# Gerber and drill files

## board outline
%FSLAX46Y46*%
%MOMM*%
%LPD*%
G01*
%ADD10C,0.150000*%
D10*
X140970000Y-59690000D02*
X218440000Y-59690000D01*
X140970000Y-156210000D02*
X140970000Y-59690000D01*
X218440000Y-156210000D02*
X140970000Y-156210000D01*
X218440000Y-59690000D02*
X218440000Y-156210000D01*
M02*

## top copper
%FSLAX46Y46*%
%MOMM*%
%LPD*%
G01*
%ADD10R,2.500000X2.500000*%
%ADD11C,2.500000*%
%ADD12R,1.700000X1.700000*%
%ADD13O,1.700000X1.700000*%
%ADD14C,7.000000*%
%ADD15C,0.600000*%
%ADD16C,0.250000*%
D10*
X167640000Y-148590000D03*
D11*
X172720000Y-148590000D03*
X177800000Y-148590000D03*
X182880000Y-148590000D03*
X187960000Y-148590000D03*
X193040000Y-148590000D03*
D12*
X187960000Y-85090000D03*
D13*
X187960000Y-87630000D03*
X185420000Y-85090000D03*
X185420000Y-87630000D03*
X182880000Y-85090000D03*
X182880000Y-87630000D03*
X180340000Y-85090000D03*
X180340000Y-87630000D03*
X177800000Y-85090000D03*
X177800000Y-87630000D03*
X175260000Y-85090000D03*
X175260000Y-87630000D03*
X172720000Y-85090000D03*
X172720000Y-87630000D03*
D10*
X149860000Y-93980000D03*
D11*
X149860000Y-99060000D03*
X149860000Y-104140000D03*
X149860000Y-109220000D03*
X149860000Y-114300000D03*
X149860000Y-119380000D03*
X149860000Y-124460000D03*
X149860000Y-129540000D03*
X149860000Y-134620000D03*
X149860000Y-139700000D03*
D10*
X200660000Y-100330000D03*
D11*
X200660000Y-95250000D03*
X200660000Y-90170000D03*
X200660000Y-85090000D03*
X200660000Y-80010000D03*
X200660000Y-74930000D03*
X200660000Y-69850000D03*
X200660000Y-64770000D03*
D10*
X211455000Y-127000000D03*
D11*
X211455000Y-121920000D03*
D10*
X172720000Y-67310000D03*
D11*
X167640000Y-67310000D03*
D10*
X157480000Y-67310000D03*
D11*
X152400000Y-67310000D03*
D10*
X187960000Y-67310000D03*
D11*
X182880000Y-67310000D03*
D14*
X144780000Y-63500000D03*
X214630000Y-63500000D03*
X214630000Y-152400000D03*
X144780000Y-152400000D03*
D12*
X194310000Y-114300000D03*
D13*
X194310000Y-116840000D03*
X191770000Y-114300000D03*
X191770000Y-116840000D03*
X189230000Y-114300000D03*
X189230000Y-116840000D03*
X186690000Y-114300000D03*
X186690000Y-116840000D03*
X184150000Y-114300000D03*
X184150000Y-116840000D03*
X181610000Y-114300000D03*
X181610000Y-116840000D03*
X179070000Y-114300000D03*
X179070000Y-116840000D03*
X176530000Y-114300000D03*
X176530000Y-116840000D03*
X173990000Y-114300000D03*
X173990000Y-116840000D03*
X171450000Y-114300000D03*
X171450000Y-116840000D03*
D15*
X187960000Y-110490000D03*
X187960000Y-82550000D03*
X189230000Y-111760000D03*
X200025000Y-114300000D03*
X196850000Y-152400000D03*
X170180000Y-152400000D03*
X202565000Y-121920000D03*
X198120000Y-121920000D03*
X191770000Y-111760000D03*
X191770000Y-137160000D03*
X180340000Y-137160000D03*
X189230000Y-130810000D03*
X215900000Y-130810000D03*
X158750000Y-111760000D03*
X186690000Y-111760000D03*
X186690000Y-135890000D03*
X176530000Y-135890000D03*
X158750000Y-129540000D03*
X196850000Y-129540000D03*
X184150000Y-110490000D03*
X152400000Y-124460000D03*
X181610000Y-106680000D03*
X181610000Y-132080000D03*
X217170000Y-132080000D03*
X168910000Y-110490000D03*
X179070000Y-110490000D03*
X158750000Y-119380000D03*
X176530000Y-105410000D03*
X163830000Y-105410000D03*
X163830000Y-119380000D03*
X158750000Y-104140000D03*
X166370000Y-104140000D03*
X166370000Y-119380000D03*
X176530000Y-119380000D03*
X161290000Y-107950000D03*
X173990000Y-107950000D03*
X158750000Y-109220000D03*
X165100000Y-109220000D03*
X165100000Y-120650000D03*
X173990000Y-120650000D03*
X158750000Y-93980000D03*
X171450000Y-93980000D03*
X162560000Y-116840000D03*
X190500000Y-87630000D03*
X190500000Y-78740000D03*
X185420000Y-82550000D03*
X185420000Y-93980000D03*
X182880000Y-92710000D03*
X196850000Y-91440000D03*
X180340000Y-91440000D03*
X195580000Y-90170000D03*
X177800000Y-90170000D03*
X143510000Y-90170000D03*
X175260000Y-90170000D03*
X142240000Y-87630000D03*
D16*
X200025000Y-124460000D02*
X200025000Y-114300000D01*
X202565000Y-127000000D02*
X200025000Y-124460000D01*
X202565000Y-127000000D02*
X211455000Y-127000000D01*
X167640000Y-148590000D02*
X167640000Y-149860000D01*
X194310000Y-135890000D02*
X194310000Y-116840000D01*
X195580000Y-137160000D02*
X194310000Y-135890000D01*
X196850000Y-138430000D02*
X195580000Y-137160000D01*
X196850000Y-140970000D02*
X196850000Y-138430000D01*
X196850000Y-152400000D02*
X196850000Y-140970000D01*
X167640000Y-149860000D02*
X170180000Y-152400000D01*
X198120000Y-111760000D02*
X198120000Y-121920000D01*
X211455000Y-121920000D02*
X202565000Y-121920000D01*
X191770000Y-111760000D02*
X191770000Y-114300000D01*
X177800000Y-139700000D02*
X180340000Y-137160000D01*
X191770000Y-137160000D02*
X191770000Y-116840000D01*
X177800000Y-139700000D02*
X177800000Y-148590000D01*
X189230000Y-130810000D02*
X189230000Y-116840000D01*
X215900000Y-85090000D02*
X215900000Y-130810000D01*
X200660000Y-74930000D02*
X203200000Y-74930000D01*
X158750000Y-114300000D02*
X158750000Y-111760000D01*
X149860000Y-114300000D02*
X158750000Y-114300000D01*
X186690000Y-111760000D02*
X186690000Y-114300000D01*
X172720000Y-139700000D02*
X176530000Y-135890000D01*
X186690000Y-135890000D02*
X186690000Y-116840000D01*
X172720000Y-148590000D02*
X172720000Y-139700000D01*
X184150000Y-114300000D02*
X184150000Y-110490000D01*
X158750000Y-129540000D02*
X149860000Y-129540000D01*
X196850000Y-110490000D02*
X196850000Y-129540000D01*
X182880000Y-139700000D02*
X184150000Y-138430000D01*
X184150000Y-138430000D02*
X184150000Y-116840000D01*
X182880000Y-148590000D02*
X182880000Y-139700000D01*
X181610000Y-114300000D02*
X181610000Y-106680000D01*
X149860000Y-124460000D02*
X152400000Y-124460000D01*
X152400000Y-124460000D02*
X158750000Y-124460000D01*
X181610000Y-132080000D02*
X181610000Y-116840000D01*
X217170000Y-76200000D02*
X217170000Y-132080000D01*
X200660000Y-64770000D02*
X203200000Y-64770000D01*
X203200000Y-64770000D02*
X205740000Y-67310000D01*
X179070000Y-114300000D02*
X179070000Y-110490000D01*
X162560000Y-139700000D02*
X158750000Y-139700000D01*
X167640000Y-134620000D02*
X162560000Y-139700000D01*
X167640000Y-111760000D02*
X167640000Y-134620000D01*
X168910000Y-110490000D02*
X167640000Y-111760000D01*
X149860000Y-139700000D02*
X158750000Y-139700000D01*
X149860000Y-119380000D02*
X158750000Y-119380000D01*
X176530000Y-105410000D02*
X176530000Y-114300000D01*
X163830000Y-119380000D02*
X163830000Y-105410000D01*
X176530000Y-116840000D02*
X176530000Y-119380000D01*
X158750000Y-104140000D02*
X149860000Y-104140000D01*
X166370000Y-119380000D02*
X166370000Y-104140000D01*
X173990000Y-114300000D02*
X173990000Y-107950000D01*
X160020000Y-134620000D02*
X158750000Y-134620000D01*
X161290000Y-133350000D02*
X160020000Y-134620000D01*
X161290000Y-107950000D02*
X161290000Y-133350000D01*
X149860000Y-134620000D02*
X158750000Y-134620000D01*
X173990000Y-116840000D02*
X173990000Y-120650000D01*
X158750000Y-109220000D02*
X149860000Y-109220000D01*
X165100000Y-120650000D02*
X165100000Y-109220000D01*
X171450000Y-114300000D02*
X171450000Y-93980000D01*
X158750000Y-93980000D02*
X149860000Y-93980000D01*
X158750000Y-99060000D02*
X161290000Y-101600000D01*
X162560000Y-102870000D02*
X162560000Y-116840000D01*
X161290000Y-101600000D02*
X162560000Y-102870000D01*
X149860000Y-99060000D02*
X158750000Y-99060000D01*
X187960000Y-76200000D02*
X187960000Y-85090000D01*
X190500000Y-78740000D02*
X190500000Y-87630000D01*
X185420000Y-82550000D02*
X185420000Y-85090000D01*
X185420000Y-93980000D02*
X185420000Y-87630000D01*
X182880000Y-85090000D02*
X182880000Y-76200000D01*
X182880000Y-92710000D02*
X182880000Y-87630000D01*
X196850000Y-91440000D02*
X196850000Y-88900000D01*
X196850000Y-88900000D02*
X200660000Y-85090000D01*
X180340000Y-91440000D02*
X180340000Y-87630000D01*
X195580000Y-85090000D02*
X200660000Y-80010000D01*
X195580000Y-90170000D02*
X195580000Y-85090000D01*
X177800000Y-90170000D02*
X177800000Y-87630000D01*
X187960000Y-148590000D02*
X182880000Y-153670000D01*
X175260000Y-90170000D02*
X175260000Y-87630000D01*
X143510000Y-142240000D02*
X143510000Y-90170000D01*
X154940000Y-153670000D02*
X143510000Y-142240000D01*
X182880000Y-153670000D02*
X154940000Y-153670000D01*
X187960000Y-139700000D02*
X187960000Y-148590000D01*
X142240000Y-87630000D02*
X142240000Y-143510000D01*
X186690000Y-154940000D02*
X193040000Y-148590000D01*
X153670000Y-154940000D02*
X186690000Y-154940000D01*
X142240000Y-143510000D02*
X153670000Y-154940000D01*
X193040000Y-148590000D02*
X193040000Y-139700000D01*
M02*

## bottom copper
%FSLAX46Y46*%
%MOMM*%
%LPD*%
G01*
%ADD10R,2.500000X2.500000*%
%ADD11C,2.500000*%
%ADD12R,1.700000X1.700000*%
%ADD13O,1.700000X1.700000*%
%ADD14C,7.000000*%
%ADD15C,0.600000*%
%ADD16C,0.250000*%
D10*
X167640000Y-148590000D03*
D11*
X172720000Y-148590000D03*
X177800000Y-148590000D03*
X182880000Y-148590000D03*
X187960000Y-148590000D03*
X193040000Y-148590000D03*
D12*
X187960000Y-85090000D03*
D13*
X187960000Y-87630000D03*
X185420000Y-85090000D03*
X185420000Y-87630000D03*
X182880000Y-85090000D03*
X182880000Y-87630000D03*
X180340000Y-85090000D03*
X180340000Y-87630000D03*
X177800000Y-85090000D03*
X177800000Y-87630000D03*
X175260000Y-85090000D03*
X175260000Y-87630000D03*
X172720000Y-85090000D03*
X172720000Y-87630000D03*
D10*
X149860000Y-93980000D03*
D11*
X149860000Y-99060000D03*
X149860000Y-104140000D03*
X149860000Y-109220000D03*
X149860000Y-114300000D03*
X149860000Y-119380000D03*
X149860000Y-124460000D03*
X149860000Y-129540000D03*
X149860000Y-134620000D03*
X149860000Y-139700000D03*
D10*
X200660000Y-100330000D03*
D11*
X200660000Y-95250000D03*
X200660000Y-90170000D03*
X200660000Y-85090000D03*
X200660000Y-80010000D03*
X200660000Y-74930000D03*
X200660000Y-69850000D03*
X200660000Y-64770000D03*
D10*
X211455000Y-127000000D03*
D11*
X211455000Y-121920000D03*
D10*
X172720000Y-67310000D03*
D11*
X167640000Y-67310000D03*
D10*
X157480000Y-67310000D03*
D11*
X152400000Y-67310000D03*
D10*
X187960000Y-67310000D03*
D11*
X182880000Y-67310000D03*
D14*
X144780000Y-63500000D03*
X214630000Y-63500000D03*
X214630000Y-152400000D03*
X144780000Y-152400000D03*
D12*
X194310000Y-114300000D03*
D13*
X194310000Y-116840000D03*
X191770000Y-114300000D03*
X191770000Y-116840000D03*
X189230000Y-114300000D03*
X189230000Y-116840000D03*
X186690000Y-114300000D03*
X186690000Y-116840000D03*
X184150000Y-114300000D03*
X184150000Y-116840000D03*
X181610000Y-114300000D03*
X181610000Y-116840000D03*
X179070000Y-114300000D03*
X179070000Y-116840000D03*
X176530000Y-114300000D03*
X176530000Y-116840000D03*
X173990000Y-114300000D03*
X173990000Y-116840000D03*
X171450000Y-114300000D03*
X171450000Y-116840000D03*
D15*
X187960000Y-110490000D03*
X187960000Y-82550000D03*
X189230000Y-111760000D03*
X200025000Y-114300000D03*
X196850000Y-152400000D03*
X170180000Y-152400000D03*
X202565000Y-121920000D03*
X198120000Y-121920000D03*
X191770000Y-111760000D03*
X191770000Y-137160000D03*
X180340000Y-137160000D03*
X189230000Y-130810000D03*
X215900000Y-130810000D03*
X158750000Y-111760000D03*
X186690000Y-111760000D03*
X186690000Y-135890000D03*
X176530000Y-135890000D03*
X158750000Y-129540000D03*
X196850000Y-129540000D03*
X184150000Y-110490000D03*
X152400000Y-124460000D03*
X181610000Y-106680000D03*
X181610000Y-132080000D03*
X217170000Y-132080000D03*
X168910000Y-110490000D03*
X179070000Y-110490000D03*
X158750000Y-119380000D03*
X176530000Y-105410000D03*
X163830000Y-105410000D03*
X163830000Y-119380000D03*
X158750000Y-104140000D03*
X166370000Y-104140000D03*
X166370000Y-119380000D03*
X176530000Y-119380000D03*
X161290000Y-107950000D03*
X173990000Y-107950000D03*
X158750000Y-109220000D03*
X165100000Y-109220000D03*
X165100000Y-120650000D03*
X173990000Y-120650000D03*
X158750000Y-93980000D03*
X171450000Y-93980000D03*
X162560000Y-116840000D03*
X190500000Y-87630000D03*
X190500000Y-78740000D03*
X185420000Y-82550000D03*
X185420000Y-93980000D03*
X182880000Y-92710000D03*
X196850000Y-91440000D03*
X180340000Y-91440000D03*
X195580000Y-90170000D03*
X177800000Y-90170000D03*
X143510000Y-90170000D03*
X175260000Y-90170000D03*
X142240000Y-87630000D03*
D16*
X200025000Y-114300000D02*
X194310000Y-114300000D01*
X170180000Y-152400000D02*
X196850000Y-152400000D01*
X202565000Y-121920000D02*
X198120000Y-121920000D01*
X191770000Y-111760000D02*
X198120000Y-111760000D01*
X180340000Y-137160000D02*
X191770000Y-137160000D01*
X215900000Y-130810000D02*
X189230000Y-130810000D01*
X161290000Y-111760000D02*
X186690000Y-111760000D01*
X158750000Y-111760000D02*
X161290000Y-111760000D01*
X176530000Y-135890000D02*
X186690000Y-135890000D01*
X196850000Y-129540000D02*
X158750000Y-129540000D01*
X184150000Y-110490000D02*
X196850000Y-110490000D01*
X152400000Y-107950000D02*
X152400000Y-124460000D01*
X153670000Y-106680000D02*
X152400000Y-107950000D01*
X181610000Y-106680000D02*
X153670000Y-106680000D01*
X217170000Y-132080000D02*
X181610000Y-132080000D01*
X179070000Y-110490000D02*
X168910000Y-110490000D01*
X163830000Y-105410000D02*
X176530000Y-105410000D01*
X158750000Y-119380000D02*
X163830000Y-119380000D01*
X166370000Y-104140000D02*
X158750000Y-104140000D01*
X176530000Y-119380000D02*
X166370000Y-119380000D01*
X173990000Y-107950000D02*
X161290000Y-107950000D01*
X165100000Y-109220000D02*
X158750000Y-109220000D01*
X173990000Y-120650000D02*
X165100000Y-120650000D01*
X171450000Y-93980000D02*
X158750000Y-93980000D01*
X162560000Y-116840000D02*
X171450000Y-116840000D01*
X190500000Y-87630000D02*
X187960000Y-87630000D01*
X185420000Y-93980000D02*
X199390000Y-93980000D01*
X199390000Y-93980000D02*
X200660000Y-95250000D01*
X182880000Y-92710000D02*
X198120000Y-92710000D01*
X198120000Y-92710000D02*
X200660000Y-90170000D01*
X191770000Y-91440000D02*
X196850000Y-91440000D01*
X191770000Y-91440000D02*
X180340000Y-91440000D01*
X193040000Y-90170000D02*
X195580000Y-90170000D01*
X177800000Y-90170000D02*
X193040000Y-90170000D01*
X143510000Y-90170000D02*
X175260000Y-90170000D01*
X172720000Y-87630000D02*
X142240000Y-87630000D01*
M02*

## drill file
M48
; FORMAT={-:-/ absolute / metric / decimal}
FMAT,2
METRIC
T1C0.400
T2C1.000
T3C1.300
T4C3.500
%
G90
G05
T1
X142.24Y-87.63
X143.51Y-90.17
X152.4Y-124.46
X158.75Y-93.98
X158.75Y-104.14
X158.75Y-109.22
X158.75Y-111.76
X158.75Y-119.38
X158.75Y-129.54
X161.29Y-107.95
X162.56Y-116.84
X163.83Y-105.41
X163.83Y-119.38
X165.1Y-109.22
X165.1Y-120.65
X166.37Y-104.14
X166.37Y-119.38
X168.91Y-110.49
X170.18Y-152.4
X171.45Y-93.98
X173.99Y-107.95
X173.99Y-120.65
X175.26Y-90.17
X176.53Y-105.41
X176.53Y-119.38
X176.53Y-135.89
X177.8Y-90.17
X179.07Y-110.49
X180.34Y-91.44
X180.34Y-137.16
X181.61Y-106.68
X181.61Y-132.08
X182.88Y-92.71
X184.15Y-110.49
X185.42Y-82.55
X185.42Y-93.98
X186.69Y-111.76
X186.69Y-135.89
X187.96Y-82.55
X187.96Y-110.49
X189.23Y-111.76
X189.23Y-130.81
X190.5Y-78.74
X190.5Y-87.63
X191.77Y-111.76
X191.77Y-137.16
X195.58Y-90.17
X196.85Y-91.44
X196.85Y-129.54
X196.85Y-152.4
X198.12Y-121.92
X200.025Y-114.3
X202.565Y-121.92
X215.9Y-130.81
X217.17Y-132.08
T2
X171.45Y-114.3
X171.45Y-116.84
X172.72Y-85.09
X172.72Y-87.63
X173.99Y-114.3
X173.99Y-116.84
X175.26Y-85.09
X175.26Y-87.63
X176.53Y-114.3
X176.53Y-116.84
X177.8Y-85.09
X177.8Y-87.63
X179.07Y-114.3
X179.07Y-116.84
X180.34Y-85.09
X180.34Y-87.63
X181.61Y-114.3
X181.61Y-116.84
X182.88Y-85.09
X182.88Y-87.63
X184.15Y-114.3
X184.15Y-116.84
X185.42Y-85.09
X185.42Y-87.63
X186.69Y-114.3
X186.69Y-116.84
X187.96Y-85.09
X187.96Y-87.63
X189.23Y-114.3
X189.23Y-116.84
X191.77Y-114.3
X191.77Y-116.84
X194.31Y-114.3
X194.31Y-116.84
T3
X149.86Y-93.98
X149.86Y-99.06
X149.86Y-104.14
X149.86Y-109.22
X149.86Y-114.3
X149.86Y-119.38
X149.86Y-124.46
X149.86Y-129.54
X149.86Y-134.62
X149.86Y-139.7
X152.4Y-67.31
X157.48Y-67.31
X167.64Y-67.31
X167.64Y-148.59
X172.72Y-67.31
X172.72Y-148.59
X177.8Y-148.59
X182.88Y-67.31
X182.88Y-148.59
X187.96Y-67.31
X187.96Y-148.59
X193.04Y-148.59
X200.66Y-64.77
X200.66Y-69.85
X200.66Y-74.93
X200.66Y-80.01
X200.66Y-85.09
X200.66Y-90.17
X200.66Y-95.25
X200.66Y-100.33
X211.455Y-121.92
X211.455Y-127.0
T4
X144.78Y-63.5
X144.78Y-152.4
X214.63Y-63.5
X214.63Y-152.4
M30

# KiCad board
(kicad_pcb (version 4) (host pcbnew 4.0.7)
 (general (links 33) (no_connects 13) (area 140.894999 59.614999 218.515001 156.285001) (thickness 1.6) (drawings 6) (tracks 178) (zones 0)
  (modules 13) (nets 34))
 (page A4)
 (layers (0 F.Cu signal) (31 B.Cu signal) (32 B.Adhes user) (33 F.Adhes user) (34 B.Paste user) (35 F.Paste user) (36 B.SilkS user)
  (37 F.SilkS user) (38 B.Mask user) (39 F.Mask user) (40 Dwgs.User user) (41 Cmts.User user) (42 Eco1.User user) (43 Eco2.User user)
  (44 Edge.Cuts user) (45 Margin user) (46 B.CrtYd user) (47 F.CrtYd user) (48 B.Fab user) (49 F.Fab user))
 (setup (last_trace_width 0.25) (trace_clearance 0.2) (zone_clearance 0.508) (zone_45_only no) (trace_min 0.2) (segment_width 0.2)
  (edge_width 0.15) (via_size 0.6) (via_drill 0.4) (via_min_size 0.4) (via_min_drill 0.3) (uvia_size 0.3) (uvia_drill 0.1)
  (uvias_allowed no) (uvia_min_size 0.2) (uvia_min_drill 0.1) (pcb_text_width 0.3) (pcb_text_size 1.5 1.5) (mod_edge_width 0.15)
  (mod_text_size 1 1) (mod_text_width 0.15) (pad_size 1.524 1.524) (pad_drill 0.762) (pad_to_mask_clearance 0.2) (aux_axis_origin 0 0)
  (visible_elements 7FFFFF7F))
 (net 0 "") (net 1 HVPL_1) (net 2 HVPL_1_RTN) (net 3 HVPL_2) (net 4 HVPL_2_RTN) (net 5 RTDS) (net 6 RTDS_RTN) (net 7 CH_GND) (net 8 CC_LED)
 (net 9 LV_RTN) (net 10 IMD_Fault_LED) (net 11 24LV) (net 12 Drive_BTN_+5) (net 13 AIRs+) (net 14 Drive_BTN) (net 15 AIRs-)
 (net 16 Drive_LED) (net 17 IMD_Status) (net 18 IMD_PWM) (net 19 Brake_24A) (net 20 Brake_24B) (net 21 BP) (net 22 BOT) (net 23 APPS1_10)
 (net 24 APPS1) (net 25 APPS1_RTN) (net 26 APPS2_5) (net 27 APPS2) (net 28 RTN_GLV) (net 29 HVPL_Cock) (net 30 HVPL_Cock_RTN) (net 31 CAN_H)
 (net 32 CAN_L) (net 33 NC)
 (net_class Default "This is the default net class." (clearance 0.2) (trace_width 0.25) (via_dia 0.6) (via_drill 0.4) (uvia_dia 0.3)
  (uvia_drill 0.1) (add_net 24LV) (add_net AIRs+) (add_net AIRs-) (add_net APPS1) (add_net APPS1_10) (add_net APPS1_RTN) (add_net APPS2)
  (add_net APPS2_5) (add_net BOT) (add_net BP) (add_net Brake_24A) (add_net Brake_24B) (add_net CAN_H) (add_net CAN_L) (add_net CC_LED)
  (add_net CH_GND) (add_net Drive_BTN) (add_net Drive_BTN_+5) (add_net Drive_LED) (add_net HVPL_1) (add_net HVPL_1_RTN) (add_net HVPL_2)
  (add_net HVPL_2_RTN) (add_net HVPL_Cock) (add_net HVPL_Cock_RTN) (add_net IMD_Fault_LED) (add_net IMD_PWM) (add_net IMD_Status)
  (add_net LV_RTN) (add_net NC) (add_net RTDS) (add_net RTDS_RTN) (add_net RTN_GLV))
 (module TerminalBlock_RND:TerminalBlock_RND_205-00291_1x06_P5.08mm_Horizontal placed (layer F.Cu) (at 167.64 148.59)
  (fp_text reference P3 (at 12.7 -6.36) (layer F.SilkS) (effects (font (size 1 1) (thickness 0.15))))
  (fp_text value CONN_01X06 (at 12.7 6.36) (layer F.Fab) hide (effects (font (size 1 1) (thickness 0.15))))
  (pad 1 thru_hole rect (at 0 0) (size 2.5 2.5) (drill 1.3) (layers *.Cu *.Mask) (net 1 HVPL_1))
  (pad 2 thru_hole circle (at 5.08 0) (size 2.5 2.5) (drill 1.3) (layers *.Cu *.Mask) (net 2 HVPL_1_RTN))
  (pad 3 thru_hole circle (at 10.16 0) (size 2.5 2.5) (drill 1.3) (layers *.Cu *.Mask) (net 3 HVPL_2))
  (pad 4 thru_hole circle (at 15.24 0) (size 2.5 2.5) (drill 1.3) (layers *.Cu *.Mask) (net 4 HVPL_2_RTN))
  (pad 5 thru_hole circle (at 20.32 0) (size 2.5 2.5) (drill 1.3) (layers *.Cu *.Mask) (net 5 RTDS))
  (pad 6 thru_hole circle (at 25.4 0) (size 2.5 2.5) (drill 1.3) (layers *.Cu *.Mask) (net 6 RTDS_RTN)))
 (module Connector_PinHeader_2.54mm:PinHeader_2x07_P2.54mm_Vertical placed (layer F.Cu) (at 187.96 85.09 270)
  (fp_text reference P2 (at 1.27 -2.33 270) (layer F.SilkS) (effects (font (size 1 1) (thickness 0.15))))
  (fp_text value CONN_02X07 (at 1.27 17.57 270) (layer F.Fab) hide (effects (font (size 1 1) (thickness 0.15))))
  (pad 1 thru_hole rect (at 0 0 270) (size 1.7 1.7) (drill 1) (layers *.Cu *.Mask) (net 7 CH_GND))
  (pad 2 thru_hole oval (at 2.54 0 270) (size 1.7 1.7) (drill 1) (layers *.Cu *.Mask) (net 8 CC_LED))
  (pad 3 thru_hole oval (at 0 2.54 270) (size 1.7 1.7) (drill 1) (layers *.Cu *.Mask) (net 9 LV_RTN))
  (pad 4 thru_hole oval (at 2.54 2.54 270) (size 1.7 1.7) (drill 1) (layers *.Cu *.Mask) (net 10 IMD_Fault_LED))
  (pad 5 thru_hole oval (at 0 5.08 270) (size 1.7 1.7) (drill 1) (layers *.Cu *.Mask) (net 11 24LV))
  (pad 6 thru_hole oval (at 2.54 5.08 270) (size 1.7 1.7) (drill 1) (layers *.Cu *.Mask) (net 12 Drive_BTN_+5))
  (pad 7 thru_hole oval (at 0 7.62 270) (size 1.7 1.7) (drill 1) (layers *.Cu *.Mask) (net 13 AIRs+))
  (pad 8 thru_hole oval (at 2.54 7.62 270) (size 1.7 1.7) (drill 1) (layers *.Cu *.Mask) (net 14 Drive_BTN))
  (pad 9 thru_hole oval (at 0 10.16 270) (size 1.7 1.7) (drill 1) (layers *.Cu *.Mask) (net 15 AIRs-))
  (pad 10 thru_hole oval (at 2.54 10.16 270) (size 1.7 1.7) (drill 1) (layers *.Cu *.Mask) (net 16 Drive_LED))
  (pad 11 thru_hole oval (at 0 12.7 270) (size 1.7 1.7) (drill 1) (layers *.Cu *.Mask) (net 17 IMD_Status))
  (pad 12 thru_hole oval (at 2.54 12.7 270) (size 1.7 1.7) (drill 1) (layers *.Cu *.Mask) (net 5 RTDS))
  (pad 13 thru_hole oval (at 0 15.24 270) (size 1.7 1.7) (drill 1) (layers *.Cu *.Mask) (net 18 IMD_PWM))
  (pad 14 thru_hole oval (at 2.54 15.24 270) (size 1.7 1.7) (drill 1) (layers *.Cu *.Mask) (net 6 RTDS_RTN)))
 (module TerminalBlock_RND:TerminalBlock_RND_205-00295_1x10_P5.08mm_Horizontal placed (layer F.Cu) (at 149.86 93.98 270)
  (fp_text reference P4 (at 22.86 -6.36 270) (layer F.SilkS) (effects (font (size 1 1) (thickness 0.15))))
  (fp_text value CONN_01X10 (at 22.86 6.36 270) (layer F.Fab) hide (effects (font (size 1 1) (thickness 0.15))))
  (pad 1 thru_hole rect (at 0 0 270) (size 2.5 2.5) (drill 1.3) (layers *.Cu *.Mask) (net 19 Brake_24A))
  (pad 2 thru_hole circle (at 5.08 0 270) (size 2.5 2.5) (drill 1.3) (layers *.Cu *.Mask) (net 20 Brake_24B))
  (pad 3 thru_hole circle (at 10.16 0 270) (size 2.5 2.5) (drill 1.3) (layers *.Cu *.Mask) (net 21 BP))
  (pad 4 thru_hole circle (at 15.24 0 270) (size 2.5 2.5) (drill 1.3) (layers *.Cu *.Mask) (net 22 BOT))
  (pad 5 thru_hole circle (at 20.32 0 270) (size 2.5 2.5) (drill 1.3) (layers *.Cu *.Mask) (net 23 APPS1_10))
  (pad 6 thru_hole circle (at 25.4 0 270) (size 2.5 2.5) (drill 1.3) (layers *.Cu *.Mask) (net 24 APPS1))
  (pad 7 thru_hole circle (at 30.48 0 270) (size 2.5 2.5) (drill 1.3) (layers *.Cu *.Mask) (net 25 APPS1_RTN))
  (pad 8 thru_hole circle (at 35.56 0 270) (size 2.5 2.5) (drill 1.3) (layers *.Cu *.Mask) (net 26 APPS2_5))
  (pad 9 thru_hole circle (at 40.64 0 270) (size 2.5 2.5) (drill 1.3) (layers *.Cu *.Mask) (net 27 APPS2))
  (pad 10 thru_hole circle (at 45.72 0 270) (size 2.5 2.5) (drill 1.3) (layers *.Cu *.Mask) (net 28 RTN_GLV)))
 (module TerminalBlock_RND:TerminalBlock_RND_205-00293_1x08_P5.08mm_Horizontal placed (layer F.Cu) (at 200.66 100.33 90)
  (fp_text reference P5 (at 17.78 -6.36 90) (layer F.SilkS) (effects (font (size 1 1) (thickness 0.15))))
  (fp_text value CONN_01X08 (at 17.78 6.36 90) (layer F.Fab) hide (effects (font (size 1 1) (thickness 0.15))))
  (pad 1 thru_hole rect (at 0 0 90) (size 2.5 2.5) (drill 1.3) (layers *.Cu *.Mask) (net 9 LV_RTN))
  (pad 2 thru_hole circle (at 5.08 0 90) (size 2.5 2.5) (drill 1.3) (layers *.Cu *.Mask) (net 10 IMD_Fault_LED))
  (pad 3 thru_hole circle (at 10.16 0 90) (size 2.5 2.5) (drill 1.3) (layers *.Cu *.Mask) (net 12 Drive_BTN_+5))
  (pad 4 thru_hole circle (at 15.24 0 90) (size 2.5 2.5) (drill 1.3) (layers *.Cu *.Mask) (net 14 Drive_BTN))
  (pad 5 thru_hole circle (at 20.32 0 90) (size 2.5 2.5) (drill 1.3) (layers *.Cu *.Mask) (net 16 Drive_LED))
  (pad 6 thru_hole circle (at 25.4 0 90) (size 2.5 2.5) (drill 1.3) (layers *.Cu *.Mask) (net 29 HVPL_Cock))
  (pad 7 thru_hole circle (at 30.48 0 90) (size 2.5 2.5) (drill 1.3) (layers *.Cu *.Mask) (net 8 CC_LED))
  (pad 8 thru_hole circle (at 35.56 0 90) (size 2.5 2.5) (drill 1.3) (layers *.Cu *.Mask) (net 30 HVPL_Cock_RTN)))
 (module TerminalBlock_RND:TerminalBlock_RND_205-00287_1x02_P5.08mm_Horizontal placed (layer F.Cu) (at 211.455 127 90)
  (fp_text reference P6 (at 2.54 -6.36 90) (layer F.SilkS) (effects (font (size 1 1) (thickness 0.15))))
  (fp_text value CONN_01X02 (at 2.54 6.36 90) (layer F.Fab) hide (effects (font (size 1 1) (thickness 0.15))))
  (pad 1 thru_hole rect (at 0 0 90) (size 2.5 2.5) (drill 1.3) (layers *.Cu *.Mask) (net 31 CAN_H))
  (pad 2 thru_hole circle (at 5.08 0 90) (size 2.5 2.5) (drill 1.3) (layers *.Cu *.Mask) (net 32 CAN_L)))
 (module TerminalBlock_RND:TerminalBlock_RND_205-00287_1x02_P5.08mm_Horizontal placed (layer F.Cu) (at 172.72 67.31 180)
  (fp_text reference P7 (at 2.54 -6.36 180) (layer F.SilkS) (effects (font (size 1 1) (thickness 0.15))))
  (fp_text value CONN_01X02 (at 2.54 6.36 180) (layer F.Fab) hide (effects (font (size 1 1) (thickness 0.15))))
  (pad 1 thru_hole rect (at 0 0 180) (size 2.5 2.5) (drill 1.3) (layers *.Cu *.Mask) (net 13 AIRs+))
  (pad 2 thru_hole circle (at 5.08 0 180) (size 2.5 2.5) (drill 1.3) (layers *.Cu *.Mask) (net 15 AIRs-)))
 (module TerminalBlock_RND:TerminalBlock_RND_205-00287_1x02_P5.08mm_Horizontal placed (layer F.Cu) (at 157.48 67.31 180)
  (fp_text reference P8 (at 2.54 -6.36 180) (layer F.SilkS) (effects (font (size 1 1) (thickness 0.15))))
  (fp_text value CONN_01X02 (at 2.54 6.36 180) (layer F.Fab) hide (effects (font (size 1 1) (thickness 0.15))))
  (pad 1 thru_hole rect (at 0 0 180) (size 2.5 2.5) (drill 1.3) (layers *.Cu *.Mask) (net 17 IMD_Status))
  (pad 2 thru_hole circle (at 5.08 0 180) (size 2.5 2.5) (drill 1.3) (layers *.Cu *.Mask) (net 18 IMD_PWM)))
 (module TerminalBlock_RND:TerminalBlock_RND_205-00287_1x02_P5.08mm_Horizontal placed (layer F.Cu) (at 187.96 67.31 180)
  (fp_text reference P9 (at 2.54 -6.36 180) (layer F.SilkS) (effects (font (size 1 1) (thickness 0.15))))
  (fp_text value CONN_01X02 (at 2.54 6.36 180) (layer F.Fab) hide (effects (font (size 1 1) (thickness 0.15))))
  (pad 1 thru_hole rect (at 0 0 180) (size 2.5 2.5) (drill 1.3) (layers *.Cu *.Mask) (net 7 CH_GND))
  (pad 2 thru_hole circle (at 5.08 0 180) (size 2.5 2.5) (drill 1.3) (layers *.Cu *.Mask) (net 11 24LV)))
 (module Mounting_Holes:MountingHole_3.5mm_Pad (layer F.Cu) (at 144.78 63.5)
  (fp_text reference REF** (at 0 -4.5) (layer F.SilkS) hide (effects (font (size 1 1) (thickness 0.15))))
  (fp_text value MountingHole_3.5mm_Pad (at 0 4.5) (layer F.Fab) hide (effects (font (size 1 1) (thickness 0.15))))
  (pad 1 thru_hole circle (at 0 0) (size 7 7) (drill 3.5) (layers *.Cu *.Mask)))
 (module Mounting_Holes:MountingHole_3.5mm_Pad (layer F.Cu) (at 214.63 63.5)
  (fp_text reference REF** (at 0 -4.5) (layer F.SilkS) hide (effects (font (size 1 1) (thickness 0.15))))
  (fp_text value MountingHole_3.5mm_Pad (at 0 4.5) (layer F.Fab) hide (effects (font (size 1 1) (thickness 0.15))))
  (pad 1 thru_hole circle (at 0 0) (size 7 7) (drill 3.5) (layers *.Cu *.Mask)))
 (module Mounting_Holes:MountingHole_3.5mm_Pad (layer F.Cu) (at 214.63 152.4)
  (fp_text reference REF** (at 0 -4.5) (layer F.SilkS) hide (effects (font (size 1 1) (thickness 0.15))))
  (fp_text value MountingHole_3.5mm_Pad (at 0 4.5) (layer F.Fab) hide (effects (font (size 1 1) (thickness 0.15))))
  (pad 1 thru_hole circle (at 0 0) (size 7 7) (drill 3.5) (layers *.Cu *.Mask)))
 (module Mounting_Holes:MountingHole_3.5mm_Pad (layer F.Cu) (at 144.78 152.4)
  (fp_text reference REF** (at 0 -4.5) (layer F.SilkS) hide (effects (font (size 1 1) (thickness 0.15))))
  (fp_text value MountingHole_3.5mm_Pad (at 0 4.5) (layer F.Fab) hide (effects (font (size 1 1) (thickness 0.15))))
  (pad 1 thru_hole circle (at 0 0) (size 7 7) (drill 3.5) (layers *.Cu *.Mask)))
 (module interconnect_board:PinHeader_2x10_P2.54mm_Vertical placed (layer F.Cu) (at 194.31 114.3 270)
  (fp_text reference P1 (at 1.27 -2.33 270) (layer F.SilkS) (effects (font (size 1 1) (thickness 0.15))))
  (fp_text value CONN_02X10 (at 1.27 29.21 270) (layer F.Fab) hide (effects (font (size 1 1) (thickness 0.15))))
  (pad 1 thru_hole rect (at 0 0 270) (size 1.7 1.7) (drill 1) (layers *.Cu *.Mask) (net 31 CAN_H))
  (pad 2 thru_hole oval (at 2.54 0 270) (size 1.7 1.7) (drill 1) (layers *.Cu *.Mask) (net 1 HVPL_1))
  (pad 3 thru_hole oval (at 0 2.54 270) (size 1.7 1.7) (drill 1) (layers *.Cu *.Mask) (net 32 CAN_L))
  (pad 4 thru_hole oval (at 2.54 2.54 270) (size 1.7 1.7) (drill 1) (layers *.Cu *.Mask) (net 3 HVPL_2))
  (pad 5 thru_hole oval (at 0 5.08 270) (size 1.7 1.7) (drill 1) (layers *.Cu *.Mask) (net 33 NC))
  (pad 6 thru_hole oval (at 2.54 5.08 270) (size 1.7 1.7) (drill 1) (layers *.Cu *.Mask) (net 29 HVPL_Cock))
  (pad 7 thru_hole oval (at 0 7.62 270) (size 1.7 1.7) (drill 1) (layers *.Cu *.Mask) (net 23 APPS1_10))
  (pad 8 thru_hole oval (at 2.54 7.62 270) (size 1.7 1.7) (drill 1) (layers *.Cu *.Mask) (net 2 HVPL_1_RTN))
  (pad 9 thru_hole oval (at 0 10.16 270) (size 1.7 1.7) (drill 1) (layers *.Cu *.Mask) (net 26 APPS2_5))
  (pad 10 thru_hole oval (at 2.54 10.16 270) (size 1.7 1.7) (drill 1) (layers *.Cu *.Mask) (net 4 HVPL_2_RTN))
  (pad 11 thru_hole oval (at 0 12.7 270) (size 1.7 1.7) (drill 1) (layers *.Cu *.Mask) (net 25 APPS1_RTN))
  (pad 12 thru_hole oval (at 2.54 12.7 270) (size 1.7 1.7) (drill 1) (layers *.Cu *.Mask) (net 30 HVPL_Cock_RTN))
  (pad 13 thru_hole oval (at 0 15.24 270) (size 1.7 1.7) (drill 1) (layers *.Cu *.Mask) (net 28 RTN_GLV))
  (pad 14 thru_hole oval (at 2.54 15.24 270) (size 1.7 1.7) (drill 1) (layers *.Cu *.Mask) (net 33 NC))
  (pad 15 thru_hole oval (at 0 17.78 270) (size 1.7 1.7) (drill 1) (layers *.Cu *.Mask) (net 24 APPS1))
  (pad 16 thru_hole oval (at 2.54 17.78 270) (size 1.7 1.7) (drill 1) (layers *.Cu *.Mask) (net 21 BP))
  (pad 17 thru_hole oval (at 0 20.32 270) (size 1.7 1.7) (drill 1) (layers *.Cu *.Mask) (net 27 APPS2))
  (pad 18 thru_hole oval (at 2.54 20.32 270) (size 1.7 1.7) (drill 1) (layers *.Cu *.Mask) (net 22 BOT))
  (pad 19 thru_hole oval (at 0 22.86 270) (size 1.7 1.7) (drill 1) (layers *.Cu *.Mask) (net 19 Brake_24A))
  (pad 20 thru_hole oval (at 2.54 22.86 270) (size 1.7 1.7) (drill 1) (layers *.Cu *.Mask) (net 20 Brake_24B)))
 (gr_line (start 140.97 59.69) (end 218.44 59.69) (angle 90) (layer Edge.Cuts) (width 0.15))
 (gr_line (start 140.97 156.21) (end 140.97 59.69) (angle 90) (layer Edge.Cuts) (width 0.15))
 (gr_line (start 218.44 156.21) (end 140.97 156.21) (angle 90) (layer Edge.Cuts) (width 0.15))
 (gr_line (start 218.44 59.69) (end 218.44 156.21) (angle 90) (layer Edge.Cuts) (width 0.15))
 (via (at 187.96 110.49) (size 0.6) (drill 0.4) (layers F.Cu B.Cu) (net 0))
 (via (at 187.96 82.55) (size 0.6) (drill 0.4) (layers F.Cu B.Cu) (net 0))
 (via (at 189.23 111.76) (size 0.6) (drill 0.4) (layers F.Cu B.Cu) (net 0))
 (segment (start 200.025 114.3) (end 194.31 114.3) (width 0.25) (layer B.Cu) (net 31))
 (via (at 200.025 114.3) (size 0.6) (drill 0.4) (layers F.Cu B.Cu) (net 31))
 (segment (start 200.025 124.46) (end 200.025 114.3) (width 0.25) (layer F.Cu) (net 31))
 (segment (start 202.565 127) (end 200.025 124.46) (width 0.25) (layer F.Cu) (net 31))
 (segment (start 202.565 127) (end 211.455 127) (width 0.25) (layer F.Cu) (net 31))
 (segment (start 167.64 148.59) (end 167.64 149.86) (width 0.25) (layer F.Cu) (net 1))
 (segment (start 194.31 135.89) (end 194.31 116.84) (width 0.25) (layer F.Cu) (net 1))
 (segment (start 195.58 137.16) (end 194.31 135.89) (width 0.25) (layer F.Cu) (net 1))
 (segment (start 196.85 138.43) (end 195.58 137.16) (width 0.25) (layer F.Cu) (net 1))
 (segment (start 196.85 140.97) (end 196.85 138.43) (width 0.25) (layer F.Cu) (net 1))
 (segment (start 196.85 152.4) (end 196.85 140.97) (width 0.25) (layer F.Cu) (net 1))
 (via (at 196.85 152.4) (size 0.6) (drill 0.4) (layers F.Cu B.Cu) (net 1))
 (segment (start 170.18 152.4) (end 196.85 152.4) (width 0.25) (layer B.Cu) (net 1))
 (via (at 170.18 152.4) (size 0.6) (drill 0.4) (layers F.Cu B.Cu) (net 1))
 (segment (start 167.64 149.86) (end 170.18 152.4) (width 0.25) (layer F.Cu) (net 1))
 (via (at 202.565 121.92) (size 0.6) (drill 0.4) (layers F.Cu B.Cu) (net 32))
 (segment (start 198.12 111.76) (end 198.12 121.92) (width 0.25) (layer F.Cu) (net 32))
 (via (at 198.12 121.92) (size 0.6) (drill 0.4) (layers F.Cu B.Cu) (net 32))
 (segment (start 202.565 121.92) (end 198.12 121.92) (width 0.25) (layer B.Cu) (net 32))
 (segment (start 211.455 121.92) (end 202.565 121.92) (width 0.25) (layer F.Cu) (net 32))
 (segment (start 191.77 111.76) (end 191.77 114.3) (width 0.25) (layer F.Cu) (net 32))
 (segment (start 191.77 111.76) (end 198.12 111.76) (width 0.25) (layer B.Cu) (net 32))
 (via (at 191.77 111.76) (size 0.6) (drill 0.4) (layers F.Cu B.Cu) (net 32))
 (segment (start 177.8 139.7) (end 180.34 137.16) (width 0.25) (layer F.Cu) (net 3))
 (segment (start 191.77 137.16) (end 191.77 116.84) (width 0.25) (layer F.Cu) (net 3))
 (via (at 191.77 137.16) (size 0.6) (drill 0.4) (layers F.Cu B.Cu) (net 3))
 (segment (start 180.34 137.16) (end 191.77 137.16) (width 0.25) (layer B.Cu) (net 3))
 (via (at 180.34 137.16) (size 0.6) (drill 0.4) (layers F.Cu B.Cu) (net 3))
 (segment (start 177.8 139.7) (end 177.8 148.59) (width 0.25) (layer F.Cu) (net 3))
 (segment (start 189.23 130.81) (end 189.23 116.84) (width 0.25) (layer F.Cu) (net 29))
 (via (at 189.23 130.81) (size 0.6) (drill 0.4) (layers F.Cu B.Cu) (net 29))
 (segment (start 215.9 130.81) (end 189.23 130.81) (width 0.25) (layer B.Cu) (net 29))
 (via (at 215.9 130.81) (size 0.6) (drill 0.4) (layers F.Cu B.Cu) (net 29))
 (segment (start 215.9 85.09) (end 215.9 130.81) (width 0.25) (layer F.Cu) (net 29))
 (segment (start 200.66 74.93) (end 203.2 74.93) (width 0.25) (layer F.Cu) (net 29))
 (segment (start 158.75 114.3) (end 158.75 111.76) (width 0.25) (layer F.Cu) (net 23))
 (via (at 158.75 111.76) (size 0.6) (drill 0.4) (layers F.Cu B.Cu) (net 23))
 (segment (start 149.86 114.3) (end 158.75 114.3) (width 0.25) (layer F.Cu) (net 23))
 (segment (start 161.29 111.76) (end 186.69 111.76) (width 0.25) (layer B.Cu) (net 23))
 (via (at 186.69 111.76) (size 0.6) (drill 0.4) (layers F.Cu B.Cu) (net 23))
 (segment (start 186.69 111.76) (end 186.69 114.3) (width 0.25) (layer F.Cu) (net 23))
 (segment (start 158.75 111.76) (end 161.29 111.76) (width 0.25) (layer B.Cu) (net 23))
 (segment (start 172.72 139.7) (end 176.53 135.89) (width 0.25) (layer F.Cu) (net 2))
 (segment (start 186.69 135.89) (end 186.69 116.84) (width 0.25) (layer F.Cu) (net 2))
 (via (at 186.69 135.89) (size 0.6) (drill 0.4) (layers F.Cu B.Cu) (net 2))
 (segment (start 176.53 135.89) (end 186.69 135.89) (width 0.25) (layer B.Cu) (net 2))
 (via (at 176.53 135.89) (size 0.6) (drill 0.4) (layers F.Cu B.Cu) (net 2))
 (segment (start 172.72 148.59) (end 172.72 139.7) (width 0.25) (layer F.Cu) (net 2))
 (segment (start 184.15 114.3) (end 184.15 110.49) (width 0.25) (layer F.Cu) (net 26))
 (segment (start 158.75 129.54) (end 149.86 129.54) (width 0.25) (layer F.Cu) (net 26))
 (via (at 158.75 129.54) (size 0.6) (drill 0.4) (layers F.Cu B.Cu) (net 26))
 (segment (start 196.85 129.54) (end 158.75 129.54) (width 0.25) (layer B.Cu) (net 26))
 (via (at 196.85 129.54) (size 0.6) (drill 0.4) (layers F.Cu B.Cu) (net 26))
 (segment (start 196.85 110.49) (end 196.85 129.54) (width 0.25) (layer F.Cu) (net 26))
 (segment (start 184.15 110.49) (end 196.85 110.49) (width 0.25) (layer B.Cu) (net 26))
 (via (at 184.15 110.49) (size 0.6) (drill 0.4) (layers F.Cu B.Cu) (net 26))
 (segment (start 182.88 139.7) (end 184.15 138.43) (width 0.25) (layer F.Cu) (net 4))
 (segment (start 184.15 138.43) (end 184.15 116.84) (width 0.25) (layer F.Cu) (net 4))
 (segment (start 182.88 148.59) (end 182.88 139.7) (width 0.25) (layer F.Cu) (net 4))
 (segment (start 181.61 114.3) (end 181.61 106.68) (width 0.25) (layer F.Cu) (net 25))
 (via (at 152.4 124.46) (size 0.6) (drill 0.4) (layers F.Cu B.Cu) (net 25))
 (segment (start 152.4 107.95) (end 152.4 124.46) (width 0.25) (layer B.Cu) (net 25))
 (segment (start 153.67 106.68) (end 152.4 107.95) (width 0.25) (layer B.Cu) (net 25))
 (segment (start 181.61 106.68) (end 153.67 106.68) (width 0.25) (layer B.Cu) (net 25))
 (via (at 181.61 106.68) (size 0.6) (drill 0.4) (layers F.Cu B.Cu) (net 25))
 (segment (start 149.86 124.46) (end 152.4 124.46) (width 0.25) (layer F.Cu) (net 25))
 (segment (start 152.4 124.46) (end 158.75 124.46) (width 0.25) (layer F.Cu) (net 25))
 (segment (start 181.61 132.08) (end 181.61 116.84) (width 0.25) (layer F.Cu) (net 30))
 (via (at 181.61 132.08) (size 0.6) (drill 0.4) (layers F.Cu B.Cu) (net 30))
 (segment (start 217.17 132.08) (end 181.61 132.08) (width 0.25) (layer B.Cu) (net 30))
 (via (at 217.17 132.08) (size 0.6) (drill 0.4) (layers F.Cu B.Cu) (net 30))
 (segment (start 217.17 76.2) (end 217.17 132.08) (width 0.25) (layer F.Cu) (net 30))
 (segment (start 200.66 64.77) (end 203.2 64.77) (width 0.25) (layer F.Cu) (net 30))
 (segment (start 203.2 64.77) (end 205.74 67.31) (width 0.25) (layer F.Cu) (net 30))
 (segment (start 179.07 114.3) (end 179.07 110.49) (width 0.25) (layer F.Cu) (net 28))
 (segment (start 162.56 139.7) (end 158.75 139.7) (width 0.25) (layer F.Cu) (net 28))
 (segment (start 167.64 134.62) (end 162.56 139.7) (width 0.25) (layer F.Cu) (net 28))
 (segment (start 167.64 111.76) (end 167.64 134.62) (width 0.25) (layer F.Cu) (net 28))
 (segment (start 168.91 110.49) (end 167.64 111.76) (width 0.25) (layer F.Cu) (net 28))
 (via (at 168.91 110.49) (size 0.6) (drill 0.4) (layers F.Cu B.Cu) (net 28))
 (segment (start 179.07 110.49) (end 168.91 110.49) (width 0.25) (layer B.Cu) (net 28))
 (via (at 179.07 110.49) (size 0.6) (drill 0.4) (layers F.Cu B.Cu) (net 28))
 (segment (start 149.86 139.7) (end 158.75 139.7) (width 0.25) (layer F.Cu) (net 28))
 (via (at 158.75 119.38) (size 0.6) (drill 0.4) (layers F.Cu B.Cu) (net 24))
 (segment (start 149.86 119.38) (end 158.75 119.38) (width 0.25) (layer F.Cu) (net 24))
 (segment (start 176.53 105.41) (end 176.53 114.3) (width 0.25) (layer F.Cu) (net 24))
 (via (at 176.53 105.41) (size 0.6) (drill 0.4) (layers F.Cu B.Cu) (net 24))
 (segment (start 163.83 105.41) (end 176.53 105.41) (width 0.25) (layer B.Cu) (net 24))
 (via (at 163.83 105.41) (size 0.6) (drill 0.4) (layers F.Cu B.Cu) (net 24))
 (segment (start 163.83 119.38) (end 163.83 105.41) (width 0.25) (layer F.Cu) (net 24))
 (via (at 163.83 119.38) (size 0.6) (drill 0.4) (layers F.Cu B.Cu) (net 24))
 (segment (start 158.75 119.38) (end 163.83 119.38) (width 0.25) (layer B.Cu) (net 24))
 (segment (start 176.53 116.84) (end 176.53 119.38) (width 0.25) (layer F.Cu) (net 21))
 (segment (start 158.75 104.14) (end 149.86 104.14) (width 0.25) (layer F.Cu) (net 21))
 (via (at 158.75 104.14) (size 0.6) (drill 0.4) (layers F.Cu B.Cu) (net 21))
 (segment (start 166.37 104.14) (end 158.75 104.14) (width 0.25) (layer B.Cu) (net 21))
 (via (at 166.37 104.14) (size 0.6) (drill 0.4) (layers F.Cu B.Cu) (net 21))
 (segment (start 166.37 119.38) (end 166.37 104.14) (width 0.25) (layer F.Cu) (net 21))
 (via (at 166.37 119.38) (size 0.6) (drill 0.4) (layers F.Cu B.Cu) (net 21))
 (segment (start 176.53 119.38) (end 166.37 119.38) (width 0.25) (layer B.Cu) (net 21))
 (via (at 176.53 119.38) (size 0.6) (drill 0.4) (layers F.Cu B.Cu) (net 21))
 (segment (start 173.99 114.3) (end 173.99 107.95) (width 0.25) (layer F.Cu) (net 27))
 (segment (start 160.02 134.62) (end 158.75 134.62) (width 0.25) (layer F.Cu) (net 27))
 (segment (start 161.29 133.35) (end 160.02 134.62) (width 0.25) (layer F.Cu) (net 27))
 (segment (start 161.29 107.95) (end 161.29 133.35) (width 0.25) (layer F.Cu) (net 27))
 (via (at 161.29 107.95) (size 0.6) (drill 0.4) (layers F.Cu B.Cu) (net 27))
 (segment (start 173.99 107.95) (end 161.29 107.95) (width 0.25) (layer B.Cu) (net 27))
 (via (at 173.99 107.95) (size 0.6) (drill 0.4) (layers F.Cu B.Cu) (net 27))
 (segment (start 149.86 134.62) (end 158.75 134.62) (width 0.25) (layer F.Cu) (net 27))
 (segment (start 173.99 116.84) (end 173.99 120.65) (width 0.25) (layer F.Cu) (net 22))
 (segment (start 158.75 109.22) (end 149.86 109.22) (width 0.25) (layer F.Cu) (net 22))
 (via (at 158.75 109.22) (size 0.6) (drill 0.4) (layers F.Cu B.Cu) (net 22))
 (segment (start 165.1 109.22) (end 158.75 109.22) (width 0.25) (layer B.Cu) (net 22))
 (via (at 165.1 109.22) (size 0.6) (drill 0.4) (layers F.Cu B.Cu) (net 22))
 (segment (start 165.1 120.65) (end 165.1 109.22) (width 0.25) (layer F.Cu) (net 22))
 (via (at 165.1 120.65) (size 0.6) (drill 0.4) (layers F.Cu B.Cu) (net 22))
 (segment (start 173.99 120.65) (end 165.1 120.65) (width 0.25) (layer B.Cu) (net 22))
 (via (at 173.99 120.65) (size 0.6) (drill 0.4) (layers F.Cu B.Cu) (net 22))
 (via (at 158.75 93.98) (size 0.6) (drill 0.4) (layers F.Cu B.Cu) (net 19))
 (segment (start 171.45 93.98) (end 158.75 93.98) (width 0.25) (layer B.Cu) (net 19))
 (via (at 171.45 93.98) (size 0.6) (drill 0.4) (layers F.Cu B.Cu) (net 19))
 (segment (start 171.45 114.3) (end 171.45 93.98) (width 0.25) (layer F.Cu) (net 19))
 (segment (start 158.75 93.98) (end 149.86 93.98) (width 0.25) (layer F.Cu) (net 19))
 (segment (start 158.75 99.06) (end 161.29 101.6) (width 0.25) (layer F.Cu) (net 20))
 (segment (start 162.56 116.84) (end 171.45 116.84) (width 0.25) (layer B.Cu) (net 20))
 (via (at 162.56 116.84) (size 0.6) (drill 0.4) (layers F.Cu B.Cu) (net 20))
 (segment (start 162.56 102.87) (end 162.56 116.84) (width 0.25) (layer F.Cu) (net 20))
 (segment (start 161.29 101.6) (end 162.56 102.87) (width 0.25) (layer F.Cu) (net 20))
 (segment (start 149.86 99.06) (end 158.75 99.06) (width 0.25) (layer F.Cu) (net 20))
 (segment (start 187.96 76.2) (end 187.96 85.09) (width 0.25) (layer F.Cu) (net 7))
 (segment (start 190.5 87.63) (end 187.96 87.63) (width 0.25) (layer B.Cu) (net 8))
 (via (at 190.5 87.63) (size 0.6) (drill 0.4) (layers F.Cu B.Cu) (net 8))
 (segment (start 190.5 78.74) (end 190.5 87.63) (width 0.25) (layer F.Cu) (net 8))
 (via (at 190.5 78.74) (size 0.6) (drill 0.4) (layers F.Cu B.Cu) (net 8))
 (via (at 185.42 82.55) (size 0.6) (drill 0.4) (layers F.Cu B.Cu) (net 9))
 (segment (start 185.42 82.55) (end 185.42 85.09) (width 0.25) (layer F.Cu) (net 9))
 (segment (start 185.42 93.98) (end 199.39 93.98) (width 0.25) (layer B.Cu) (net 10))
 (segment (start 199.39 93.98) (end 200.66 95.25) (width 0.25) (layer B.Cu) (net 10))
 (segment (start 185.42 93.98) (end 185.42 87.63) (width 0.25) (layer F.Cu) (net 10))
 (via (at 185.42 93.98) (size 0.6) (drill 0.4) (layers F.Cu B.Cu) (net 10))
 (segment (start 182.88 85.09) (end 182.88 76.2) (width 0.25) (layer F.Cu) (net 11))
 (segment (start 182.88 92.71) (end 198.12 92.71) (width 0.25) (layer B.Cu) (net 12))
 (segment (start 198.12 92.71) (end 200.66 90.17) (width 0.25) (layer B.Cu) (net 12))
 (segment (start 182.88 92.71) (end 182.88 87.63) (width 0.25) (layer F.Cu) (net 12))
 (via (at 182.88 92.71) (size 0.6) (drill 0.4) (layers F.Cu B.Cu) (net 12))
 (segment (start 196.85 91.44) (end 196.85 88.9) (width 0.25) (layer F.Cu) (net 14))
 (segment (start 196.85 88.9) (end 200.66 85.09) (width 0.25) (layer F.Cu) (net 14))
 (segment (start 191.77 91.44) (end 196.85 91.44) (width 0.25) (layer B.Cu) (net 14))
 (via (at 196.85 91.44) (size 0.6) (drill 0.4) (layers F.Cu B.Cu) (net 14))
 (segment (start 191.77 91.44) (end 180.34 91.44) (width 0.25) (layer B.Cu) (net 14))
 (segment (start 180.34 91.44) (end 180.34 87.63) (width 0.25) (layer F.Cu) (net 14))
 (via (at 180.34 91.44) (size 0.6) (drill 0.4) (layers F.Cu B.Cu) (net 14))
 (segment (start 195.58 85.09) (end 200.66 80.01) (width 0.25) (layer F.Cu) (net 16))
 (segment (start 195.58 90.17) (end 195.58 85.09) (width 0.25) (layer F.Cu) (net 16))
 (segment (start 193.04 90.17) (end 195.58 90.17) (width 0.25) (layer B.Cu) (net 16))
 (via (at 195.58 90.17) (size 0.6) (drill 0.4) (layers F.Cu B.Cu) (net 16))
 (segment (start 177.8 90.17) (end 193.04 90.17) (width 0.25) (layer B.Cu) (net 16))
 (segment (start 177.8 90.17) (end 177.8 87.63) (width 0.25) (layer F.Cu) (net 16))
 (via (at 177.8 90.17) (size 0.6) (drill 0.4) (layers F.Cu B.Cu) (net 16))
 (segment (start 187.96 148.59) (end 182.88 153.67) (width 0.25) (layer F.Cu) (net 5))
 (via (at 143.51 90.17) (size 0.6) (drill 0.4) (layers F.Cu B.Cu) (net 5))
 (segment (start 143.51 90.17) (end 175.26 90.17) (width 0.25) (layer B.Cu) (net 5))
 (via (at 175.26 90.17) (size 0.6) (drill 0.4) (layers F.Cu B.Cu) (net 5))
 (segment (start 175.26 90.17) (end 175.26 87.63) (width 0.25) (layer F.Cu) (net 5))
 (segment (start 143.51 142.24) (end 143.51 90.17) (width 0.25) (layer F.Cu) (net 5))
 (segment (start 154.94 153.67) (end 143.51 142.24) (width 0.25) (layer F.Cu) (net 5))
 (segment (start 182.88 153.67) (end 154.94 153.67) (width 0.25) (layer F.Cu) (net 5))
 (segment (start 187.96 139.7) (end 187.96 148.59) (width 0.25) (layer F.Cu) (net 5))
 (segment (start 142.24 87.63) (end 142.24 143.51) (width 0.25) (layer F.Cu) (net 6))
 (segment (start 172.72 87.63) (end 142.24 87.63) (width 0.25) (layer B.Cu) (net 6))
 (via (at 142.24 87.63) (size 0.6) (drill 0.4) (layers F.Cu B.Cu) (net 6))
 (segment (start 186.69 154.94) (end 193.04 148.59) (width 0.25) (layer F.Cu) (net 6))
 (segment (start 153.67 154.94) (end 186.69 154.94) (width 0.25) (layer F.Cu) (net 6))
 (segment (start 142.24 143.51) (end 153.67 154.94) (width 0.25) (layer F.Cu) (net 6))
 (segment (start 193.04 148.59) (end 193.04 139.7) (width 0.25) (layer F.Cu) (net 6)))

